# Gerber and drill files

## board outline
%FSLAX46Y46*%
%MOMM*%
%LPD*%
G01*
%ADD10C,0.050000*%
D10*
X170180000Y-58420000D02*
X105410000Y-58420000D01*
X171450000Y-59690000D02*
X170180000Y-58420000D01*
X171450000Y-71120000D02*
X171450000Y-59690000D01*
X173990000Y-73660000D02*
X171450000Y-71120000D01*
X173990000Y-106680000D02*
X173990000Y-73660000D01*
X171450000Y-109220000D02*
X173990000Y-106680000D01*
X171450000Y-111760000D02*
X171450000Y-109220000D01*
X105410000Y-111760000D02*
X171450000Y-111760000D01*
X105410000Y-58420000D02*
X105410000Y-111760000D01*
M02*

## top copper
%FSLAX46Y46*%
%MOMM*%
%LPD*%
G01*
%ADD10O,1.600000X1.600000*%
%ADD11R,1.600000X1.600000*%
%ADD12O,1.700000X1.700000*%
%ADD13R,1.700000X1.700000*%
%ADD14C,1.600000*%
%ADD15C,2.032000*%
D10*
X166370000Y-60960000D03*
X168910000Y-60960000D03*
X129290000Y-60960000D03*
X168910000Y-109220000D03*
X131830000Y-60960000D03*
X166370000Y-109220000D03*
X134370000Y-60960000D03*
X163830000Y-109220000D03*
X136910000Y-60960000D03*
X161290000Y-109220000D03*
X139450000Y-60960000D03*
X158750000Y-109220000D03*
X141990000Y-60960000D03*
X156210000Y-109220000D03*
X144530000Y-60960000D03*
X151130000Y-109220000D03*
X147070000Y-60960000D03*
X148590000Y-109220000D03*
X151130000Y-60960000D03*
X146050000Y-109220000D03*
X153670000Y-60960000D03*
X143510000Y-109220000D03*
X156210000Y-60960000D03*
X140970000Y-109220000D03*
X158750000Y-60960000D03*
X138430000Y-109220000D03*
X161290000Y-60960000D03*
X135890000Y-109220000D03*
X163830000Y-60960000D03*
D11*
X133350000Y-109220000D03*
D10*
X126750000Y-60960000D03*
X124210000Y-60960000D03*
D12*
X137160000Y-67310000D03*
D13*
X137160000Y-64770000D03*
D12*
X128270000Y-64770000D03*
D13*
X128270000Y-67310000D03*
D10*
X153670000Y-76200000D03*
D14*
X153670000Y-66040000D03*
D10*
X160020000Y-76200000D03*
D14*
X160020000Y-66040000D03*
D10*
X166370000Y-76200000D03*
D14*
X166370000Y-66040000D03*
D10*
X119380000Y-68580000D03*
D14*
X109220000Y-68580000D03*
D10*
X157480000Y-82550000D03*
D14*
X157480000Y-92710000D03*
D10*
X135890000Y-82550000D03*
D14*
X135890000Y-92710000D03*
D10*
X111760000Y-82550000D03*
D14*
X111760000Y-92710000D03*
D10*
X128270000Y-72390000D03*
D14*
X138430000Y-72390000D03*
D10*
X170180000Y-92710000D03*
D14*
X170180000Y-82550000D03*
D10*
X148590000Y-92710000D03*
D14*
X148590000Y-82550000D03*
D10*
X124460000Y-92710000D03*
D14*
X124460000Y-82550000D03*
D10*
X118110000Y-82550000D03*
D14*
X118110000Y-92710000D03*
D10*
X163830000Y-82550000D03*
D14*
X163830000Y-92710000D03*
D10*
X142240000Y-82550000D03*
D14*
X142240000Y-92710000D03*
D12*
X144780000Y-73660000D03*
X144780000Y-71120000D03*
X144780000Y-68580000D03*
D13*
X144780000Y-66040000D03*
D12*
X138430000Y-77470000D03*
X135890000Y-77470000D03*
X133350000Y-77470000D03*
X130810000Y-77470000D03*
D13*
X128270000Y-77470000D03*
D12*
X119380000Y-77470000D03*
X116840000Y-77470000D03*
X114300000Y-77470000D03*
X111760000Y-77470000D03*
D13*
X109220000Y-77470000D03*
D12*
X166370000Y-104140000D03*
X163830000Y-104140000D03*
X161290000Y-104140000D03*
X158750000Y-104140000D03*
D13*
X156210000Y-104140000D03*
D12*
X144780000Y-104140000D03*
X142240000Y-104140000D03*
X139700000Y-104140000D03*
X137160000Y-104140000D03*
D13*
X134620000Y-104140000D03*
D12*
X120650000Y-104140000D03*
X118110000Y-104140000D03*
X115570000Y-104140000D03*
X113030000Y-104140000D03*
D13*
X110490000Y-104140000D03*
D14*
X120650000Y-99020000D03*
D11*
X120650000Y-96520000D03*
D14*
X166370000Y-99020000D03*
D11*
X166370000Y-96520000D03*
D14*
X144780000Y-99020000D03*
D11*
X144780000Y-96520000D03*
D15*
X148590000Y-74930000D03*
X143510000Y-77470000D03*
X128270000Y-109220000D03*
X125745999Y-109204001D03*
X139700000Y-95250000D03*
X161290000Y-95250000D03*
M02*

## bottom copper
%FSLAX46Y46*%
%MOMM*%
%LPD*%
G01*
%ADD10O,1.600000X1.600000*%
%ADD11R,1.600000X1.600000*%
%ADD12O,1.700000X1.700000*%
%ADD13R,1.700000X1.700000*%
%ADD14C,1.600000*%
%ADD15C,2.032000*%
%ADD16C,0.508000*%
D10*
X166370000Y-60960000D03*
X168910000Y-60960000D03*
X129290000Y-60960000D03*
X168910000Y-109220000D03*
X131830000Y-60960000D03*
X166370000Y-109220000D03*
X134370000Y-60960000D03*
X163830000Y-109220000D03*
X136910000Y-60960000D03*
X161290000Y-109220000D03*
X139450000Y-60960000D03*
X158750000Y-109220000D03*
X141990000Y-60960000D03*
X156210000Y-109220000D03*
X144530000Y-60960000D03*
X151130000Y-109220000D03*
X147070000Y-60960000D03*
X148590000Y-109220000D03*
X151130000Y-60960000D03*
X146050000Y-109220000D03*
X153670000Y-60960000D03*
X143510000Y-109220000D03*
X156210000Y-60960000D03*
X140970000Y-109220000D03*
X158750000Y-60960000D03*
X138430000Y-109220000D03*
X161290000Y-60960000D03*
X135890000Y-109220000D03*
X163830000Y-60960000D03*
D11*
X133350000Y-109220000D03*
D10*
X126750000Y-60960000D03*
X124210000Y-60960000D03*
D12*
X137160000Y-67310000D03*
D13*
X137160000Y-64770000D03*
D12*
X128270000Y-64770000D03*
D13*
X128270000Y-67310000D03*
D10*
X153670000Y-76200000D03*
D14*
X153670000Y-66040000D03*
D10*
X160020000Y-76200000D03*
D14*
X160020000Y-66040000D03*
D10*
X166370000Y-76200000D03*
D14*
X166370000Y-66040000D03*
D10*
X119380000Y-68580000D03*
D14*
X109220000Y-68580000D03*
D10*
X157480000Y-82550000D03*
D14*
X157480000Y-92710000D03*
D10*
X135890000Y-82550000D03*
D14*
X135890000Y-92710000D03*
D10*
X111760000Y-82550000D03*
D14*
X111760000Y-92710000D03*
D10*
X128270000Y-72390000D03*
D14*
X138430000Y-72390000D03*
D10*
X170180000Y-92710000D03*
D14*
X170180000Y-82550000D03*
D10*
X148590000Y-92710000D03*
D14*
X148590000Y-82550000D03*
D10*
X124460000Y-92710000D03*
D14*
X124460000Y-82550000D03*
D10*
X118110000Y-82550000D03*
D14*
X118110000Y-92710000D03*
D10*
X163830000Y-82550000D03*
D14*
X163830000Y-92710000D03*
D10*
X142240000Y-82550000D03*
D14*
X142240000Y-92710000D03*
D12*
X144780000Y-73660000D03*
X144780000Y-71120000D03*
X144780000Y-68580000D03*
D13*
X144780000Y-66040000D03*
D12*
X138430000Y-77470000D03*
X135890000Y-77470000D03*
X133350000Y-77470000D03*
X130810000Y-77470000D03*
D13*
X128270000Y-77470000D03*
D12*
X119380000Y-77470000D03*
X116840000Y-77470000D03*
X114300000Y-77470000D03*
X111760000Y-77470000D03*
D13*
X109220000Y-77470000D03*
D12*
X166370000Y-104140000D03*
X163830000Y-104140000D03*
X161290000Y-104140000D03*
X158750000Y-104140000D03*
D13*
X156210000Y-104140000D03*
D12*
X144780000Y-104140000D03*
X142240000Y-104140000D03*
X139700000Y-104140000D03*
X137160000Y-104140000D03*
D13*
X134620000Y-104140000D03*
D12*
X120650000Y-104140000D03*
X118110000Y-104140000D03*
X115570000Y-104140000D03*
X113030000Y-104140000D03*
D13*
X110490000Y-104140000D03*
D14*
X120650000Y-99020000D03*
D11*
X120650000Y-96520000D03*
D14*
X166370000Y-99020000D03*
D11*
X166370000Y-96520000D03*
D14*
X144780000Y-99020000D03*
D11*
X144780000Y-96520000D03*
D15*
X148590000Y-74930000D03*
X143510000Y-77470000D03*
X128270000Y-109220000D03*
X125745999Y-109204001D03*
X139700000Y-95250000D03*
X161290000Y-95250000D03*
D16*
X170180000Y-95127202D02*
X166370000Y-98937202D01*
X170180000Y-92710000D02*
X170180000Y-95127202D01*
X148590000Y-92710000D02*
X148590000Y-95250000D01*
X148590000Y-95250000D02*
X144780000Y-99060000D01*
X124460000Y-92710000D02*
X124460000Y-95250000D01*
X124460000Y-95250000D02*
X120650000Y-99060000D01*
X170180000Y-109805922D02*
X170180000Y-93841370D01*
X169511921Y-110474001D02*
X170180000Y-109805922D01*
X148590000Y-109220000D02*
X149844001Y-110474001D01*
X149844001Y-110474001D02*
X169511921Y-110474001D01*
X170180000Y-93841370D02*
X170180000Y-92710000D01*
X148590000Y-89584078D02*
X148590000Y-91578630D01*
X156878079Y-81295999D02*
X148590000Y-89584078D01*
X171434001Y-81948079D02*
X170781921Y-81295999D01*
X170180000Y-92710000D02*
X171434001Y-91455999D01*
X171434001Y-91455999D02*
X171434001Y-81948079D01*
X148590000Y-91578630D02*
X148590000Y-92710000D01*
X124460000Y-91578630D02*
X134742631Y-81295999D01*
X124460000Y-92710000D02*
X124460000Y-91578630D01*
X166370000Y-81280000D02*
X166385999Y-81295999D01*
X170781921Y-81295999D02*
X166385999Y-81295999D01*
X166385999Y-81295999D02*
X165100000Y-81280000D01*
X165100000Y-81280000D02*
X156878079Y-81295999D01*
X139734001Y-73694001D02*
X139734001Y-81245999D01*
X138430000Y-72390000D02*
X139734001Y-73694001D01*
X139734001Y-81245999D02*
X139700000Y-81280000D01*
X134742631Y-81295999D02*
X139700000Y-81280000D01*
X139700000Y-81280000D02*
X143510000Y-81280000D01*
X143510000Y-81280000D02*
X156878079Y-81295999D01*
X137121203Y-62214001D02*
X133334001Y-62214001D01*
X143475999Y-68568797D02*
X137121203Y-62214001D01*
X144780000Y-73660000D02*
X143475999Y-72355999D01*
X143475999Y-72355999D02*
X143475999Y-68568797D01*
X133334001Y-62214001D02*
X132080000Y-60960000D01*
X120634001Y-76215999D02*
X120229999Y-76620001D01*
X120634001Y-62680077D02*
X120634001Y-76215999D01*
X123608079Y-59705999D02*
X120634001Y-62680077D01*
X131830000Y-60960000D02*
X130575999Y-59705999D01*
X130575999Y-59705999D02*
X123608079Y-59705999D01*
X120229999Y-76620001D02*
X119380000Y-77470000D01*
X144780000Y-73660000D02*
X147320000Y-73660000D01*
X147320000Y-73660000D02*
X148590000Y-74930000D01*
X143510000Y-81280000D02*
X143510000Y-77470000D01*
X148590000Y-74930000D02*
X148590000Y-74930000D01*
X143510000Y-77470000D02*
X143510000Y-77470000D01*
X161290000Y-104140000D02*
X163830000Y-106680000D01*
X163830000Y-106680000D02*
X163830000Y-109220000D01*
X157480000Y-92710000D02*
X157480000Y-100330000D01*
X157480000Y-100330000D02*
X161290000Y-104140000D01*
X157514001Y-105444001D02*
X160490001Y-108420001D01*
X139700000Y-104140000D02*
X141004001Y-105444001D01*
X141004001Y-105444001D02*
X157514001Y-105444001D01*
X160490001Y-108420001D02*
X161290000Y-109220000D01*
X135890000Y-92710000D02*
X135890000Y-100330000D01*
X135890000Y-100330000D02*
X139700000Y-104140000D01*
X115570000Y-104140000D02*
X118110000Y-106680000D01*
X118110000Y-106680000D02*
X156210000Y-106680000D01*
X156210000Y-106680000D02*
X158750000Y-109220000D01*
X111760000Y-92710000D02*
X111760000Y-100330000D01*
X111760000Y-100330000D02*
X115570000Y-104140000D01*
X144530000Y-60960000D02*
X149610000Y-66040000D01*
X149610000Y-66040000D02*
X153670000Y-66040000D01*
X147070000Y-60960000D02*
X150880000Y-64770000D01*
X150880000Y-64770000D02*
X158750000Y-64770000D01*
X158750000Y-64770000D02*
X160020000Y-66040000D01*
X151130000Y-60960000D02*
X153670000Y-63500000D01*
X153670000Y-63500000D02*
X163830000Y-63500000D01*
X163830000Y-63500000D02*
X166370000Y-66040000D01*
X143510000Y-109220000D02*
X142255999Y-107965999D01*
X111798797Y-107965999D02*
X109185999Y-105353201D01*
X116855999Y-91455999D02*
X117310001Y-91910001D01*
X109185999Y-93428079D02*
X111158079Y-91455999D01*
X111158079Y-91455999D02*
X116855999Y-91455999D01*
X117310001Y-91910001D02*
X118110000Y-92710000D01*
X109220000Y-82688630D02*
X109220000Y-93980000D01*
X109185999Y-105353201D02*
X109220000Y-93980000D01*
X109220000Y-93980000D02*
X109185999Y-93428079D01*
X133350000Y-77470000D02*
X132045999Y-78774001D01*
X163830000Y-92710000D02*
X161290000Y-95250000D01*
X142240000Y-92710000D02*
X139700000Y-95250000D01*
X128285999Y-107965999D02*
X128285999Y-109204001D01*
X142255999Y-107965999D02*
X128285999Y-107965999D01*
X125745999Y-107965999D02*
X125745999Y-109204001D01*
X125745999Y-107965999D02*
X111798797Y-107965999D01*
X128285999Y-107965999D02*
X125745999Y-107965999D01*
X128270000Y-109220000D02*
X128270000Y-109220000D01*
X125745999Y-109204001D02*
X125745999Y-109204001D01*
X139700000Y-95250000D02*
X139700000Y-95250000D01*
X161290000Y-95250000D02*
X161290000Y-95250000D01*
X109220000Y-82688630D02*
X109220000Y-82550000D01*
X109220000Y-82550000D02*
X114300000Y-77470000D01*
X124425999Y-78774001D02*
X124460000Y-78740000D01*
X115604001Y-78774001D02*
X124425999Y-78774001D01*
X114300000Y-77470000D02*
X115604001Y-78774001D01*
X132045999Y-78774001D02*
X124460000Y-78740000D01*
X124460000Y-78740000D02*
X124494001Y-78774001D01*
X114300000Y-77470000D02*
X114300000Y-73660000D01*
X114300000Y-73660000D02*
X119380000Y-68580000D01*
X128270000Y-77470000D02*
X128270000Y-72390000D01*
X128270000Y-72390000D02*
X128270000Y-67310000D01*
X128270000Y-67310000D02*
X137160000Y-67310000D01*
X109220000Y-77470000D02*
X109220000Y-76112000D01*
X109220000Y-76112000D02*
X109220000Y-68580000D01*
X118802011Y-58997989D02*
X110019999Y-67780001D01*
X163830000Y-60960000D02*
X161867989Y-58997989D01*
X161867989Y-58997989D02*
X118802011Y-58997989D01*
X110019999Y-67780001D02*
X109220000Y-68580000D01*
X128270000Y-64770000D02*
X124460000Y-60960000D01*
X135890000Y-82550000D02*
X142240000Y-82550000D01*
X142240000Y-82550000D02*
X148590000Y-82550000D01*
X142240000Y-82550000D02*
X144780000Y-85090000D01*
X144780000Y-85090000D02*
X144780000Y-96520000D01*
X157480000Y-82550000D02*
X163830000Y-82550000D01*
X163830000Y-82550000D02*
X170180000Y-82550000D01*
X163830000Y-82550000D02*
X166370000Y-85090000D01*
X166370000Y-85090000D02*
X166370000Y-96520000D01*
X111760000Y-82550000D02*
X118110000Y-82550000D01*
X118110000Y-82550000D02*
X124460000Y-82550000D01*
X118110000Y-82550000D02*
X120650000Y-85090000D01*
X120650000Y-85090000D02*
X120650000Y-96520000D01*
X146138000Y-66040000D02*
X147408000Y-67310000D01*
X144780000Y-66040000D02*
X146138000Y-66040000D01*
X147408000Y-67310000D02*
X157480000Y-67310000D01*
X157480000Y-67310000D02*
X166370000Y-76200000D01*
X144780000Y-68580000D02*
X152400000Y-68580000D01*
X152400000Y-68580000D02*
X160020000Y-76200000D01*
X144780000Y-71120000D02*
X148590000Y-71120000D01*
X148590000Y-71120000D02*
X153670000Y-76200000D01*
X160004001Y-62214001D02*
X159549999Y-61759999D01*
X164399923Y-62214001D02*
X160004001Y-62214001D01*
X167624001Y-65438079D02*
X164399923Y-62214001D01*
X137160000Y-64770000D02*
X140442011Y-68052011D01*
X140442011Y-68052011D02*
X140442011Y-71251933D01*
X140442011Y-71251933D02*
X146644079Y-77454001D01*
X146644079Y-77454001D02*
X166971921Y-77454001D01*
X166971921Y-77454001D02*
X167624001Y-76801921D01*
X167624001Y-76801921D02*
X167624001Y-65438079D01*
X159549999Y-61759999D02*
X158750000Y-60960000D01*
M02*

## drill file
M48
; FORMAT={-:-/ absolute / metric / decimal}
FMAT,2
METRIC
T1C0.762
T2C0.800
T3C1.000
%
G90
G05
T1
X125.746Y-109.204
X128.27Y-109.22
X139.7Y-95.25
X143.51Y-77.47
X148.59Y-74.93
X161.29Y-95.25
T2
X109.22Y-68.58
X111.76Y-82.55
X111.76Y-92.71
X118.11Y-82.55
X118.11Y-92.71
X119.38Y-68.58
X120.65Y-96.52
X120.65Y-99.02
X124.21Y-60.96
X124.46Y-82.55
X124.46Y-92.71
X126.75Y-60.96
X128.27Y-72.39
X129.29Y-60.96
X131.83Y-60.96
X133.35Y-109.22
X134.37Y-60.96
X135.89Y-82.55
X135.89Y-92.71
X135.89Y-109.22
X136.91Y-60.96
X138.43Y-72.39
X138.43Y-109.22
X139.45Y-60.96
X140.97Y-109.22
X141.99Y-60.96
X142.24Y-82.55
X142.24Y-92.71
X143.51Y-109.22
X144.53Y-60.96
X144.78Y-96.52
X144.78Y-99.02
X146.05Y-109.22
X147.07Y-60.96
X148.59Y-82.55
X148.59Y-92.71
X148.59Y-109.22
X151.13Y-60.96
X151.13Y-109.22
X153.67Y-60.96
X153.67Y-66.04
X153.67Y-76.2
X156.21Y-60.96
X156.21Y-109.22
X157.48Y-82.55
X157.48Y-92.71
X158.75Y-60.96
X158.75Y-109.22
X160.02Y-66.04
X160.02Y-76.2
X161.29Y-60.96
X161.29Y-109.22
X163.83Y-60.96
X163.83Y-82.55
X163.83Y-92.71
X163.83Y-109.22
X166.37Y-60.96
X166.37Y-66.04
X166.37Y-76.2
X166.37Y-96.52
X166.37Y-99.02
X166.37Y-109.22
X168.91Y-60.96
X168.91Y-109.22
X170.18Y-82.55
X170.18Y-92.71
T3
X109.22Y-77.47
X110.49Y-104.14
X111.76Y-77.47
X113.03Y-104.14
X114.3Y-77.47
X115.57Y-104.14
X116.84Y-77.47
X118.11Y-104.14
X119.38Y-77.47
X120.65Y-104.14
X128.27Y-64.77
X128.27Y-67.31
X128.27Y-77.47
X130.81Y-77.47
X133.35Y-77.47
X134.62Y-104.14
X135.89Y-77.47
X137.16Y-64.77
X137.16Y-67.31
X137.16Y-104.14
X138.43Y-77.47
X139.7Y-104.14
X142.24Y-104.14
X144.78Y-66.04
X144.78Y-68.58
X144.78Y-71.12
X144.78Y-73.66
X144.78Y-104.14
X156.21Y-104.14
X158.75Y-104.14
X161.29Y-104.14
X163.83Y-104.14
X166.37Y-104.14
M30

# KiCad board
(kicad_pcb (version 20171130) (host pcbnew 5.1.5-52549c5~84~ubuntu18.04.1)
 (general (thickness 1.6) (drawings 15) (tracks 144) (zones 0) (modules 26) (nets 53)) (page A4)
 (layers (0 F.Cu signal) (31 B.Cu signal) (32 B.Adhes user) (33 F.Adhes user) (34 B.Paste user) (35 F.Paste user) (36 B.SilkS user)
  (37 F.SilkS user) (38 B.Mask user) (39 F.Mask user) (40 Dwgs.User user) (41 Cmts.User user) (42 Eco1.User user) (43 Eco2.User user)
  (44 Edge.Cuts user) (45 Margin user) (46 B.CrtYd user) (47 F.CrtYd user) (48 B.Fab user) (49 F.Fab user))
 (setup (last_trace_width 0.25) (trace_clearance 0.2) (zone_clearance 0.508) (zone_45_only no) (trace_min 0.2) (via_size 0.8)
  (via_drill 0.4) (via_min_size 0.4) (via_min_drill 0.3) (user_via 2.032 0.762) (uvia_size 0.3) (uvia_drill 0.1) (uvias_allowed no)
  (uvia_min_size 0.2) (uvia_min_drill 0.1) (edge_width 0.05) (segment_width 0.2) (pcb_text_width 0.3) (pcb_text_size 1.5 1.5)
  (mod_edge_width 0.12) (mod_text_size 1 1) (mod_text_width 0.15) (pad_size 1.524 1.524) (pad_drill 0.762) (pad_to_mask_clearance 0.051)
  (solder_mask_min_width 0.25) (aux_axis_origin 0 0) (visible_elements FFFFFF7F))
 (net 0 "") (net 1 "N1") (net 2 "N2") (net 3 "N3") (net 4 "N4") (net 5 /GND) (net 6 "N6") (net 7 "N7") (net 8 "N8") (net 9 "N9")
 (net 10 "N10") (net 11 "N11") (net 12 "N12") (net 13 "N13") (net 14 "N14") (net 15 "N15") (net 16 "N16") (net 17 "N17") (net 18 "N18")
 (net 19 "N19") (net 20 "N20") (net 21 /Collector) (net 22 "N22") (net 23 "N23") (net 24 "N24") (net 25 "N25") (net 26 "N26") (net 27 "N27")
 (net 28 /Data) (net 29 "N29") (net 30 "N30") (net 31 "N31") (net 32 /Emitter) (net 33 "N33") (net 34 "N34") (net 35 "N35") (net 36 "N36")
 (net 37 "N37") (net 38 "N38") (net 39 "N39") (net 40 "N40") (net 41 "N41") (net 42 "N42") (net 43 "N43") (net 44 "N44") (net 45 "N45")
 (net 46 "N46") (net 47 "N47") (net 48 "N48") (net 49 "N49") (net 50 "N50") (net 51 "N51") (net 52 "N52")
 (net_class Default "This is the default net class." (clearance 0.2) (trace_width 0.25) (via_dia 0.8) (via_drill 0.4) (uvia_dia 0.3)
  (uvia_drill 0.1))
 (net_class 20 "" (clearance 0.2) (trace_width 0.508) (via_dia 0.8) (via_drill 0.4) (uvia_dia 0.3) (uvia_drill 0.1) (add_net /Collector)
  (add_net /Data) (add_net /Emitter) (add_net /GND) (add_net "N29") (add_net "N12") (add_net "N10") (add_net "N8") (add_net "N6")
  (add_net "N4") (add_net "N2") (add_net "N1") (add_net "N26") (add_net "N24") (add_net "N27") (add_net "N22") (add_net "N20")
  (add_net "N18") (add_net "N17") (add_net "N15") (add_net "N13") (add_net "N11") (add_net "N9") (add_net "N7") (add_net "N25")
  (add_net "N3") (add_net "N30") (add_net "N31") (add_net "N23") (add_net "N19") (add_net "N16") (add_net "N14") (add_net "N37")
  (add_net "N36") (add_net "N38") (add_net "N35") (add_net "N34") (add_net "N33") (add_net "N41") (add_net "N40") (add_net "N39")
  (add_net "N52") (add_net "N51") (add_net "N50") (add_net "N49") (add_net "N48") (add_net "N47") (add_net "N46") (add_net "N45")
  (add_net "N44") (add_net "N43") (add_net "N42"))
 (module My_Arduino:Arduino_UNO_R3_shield (layer F.Cu) (at 133.35 109.22)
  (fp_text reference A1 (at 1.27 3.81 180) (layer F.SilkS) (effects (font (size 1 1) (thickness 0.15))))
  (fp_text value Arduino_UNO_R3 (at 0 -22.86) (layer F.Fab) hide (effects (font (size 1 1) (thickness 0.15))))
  (pad 16 thru_hole oval (at 33.02 -48.26 270) (size 1.6 1.6) (drill 0.8) (layers *.Cu *.Mask) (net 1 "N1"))
  (pad 15 thru_hole oval (at 35.56 -48.26 270) (size 1.6 1.6) (drill 0.8) (layers *.Cu *.Mask) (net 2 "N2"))
  (pad 30 thru_hole oval (at -4.06 -48.26 270) (size 1.6 1.6) (drill 0.8) (layers *.Cu *.Mask) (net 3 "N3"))
  (pad 14 thru_hole oval (at 35.56 0 270) (size 1.6 1.6) (drill 0.8) (layers *.Cu *.Mask) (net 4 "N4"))
  (pad 29 thru_hole oval (at -1.52 -48.26 270) (size 1.6 1.6) (drill 0.8) (layers *.Cu *.Mask) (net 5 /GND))
  (pad 13 thru_hole oval (at 33.02 0 270) (size 1.6 1.6) (drill 0.8) (layers *.Cu *.Mask) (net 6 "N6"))
  (pad 28 thru_hole oval (at 1.02 -48.26 270) (size 1.6 1.6) (drill 0.8) (layers *.Cu *.Mask) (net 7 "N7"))
  (pad 12 thru_hole oval (at 30.48 0 270) (size 1.6 1.6) (drill 0.8) (layers *.Cu *.Mask) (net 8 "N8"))
  (pad 27 thru_hole oval (at 3.56 -48.26 270) (size 1.6 1.6) (drill 0.8) (layers *.Cu *.Mask) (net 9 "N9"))
  (pad 11 thru_hole oval (at 27.94 0 270) (size 1.6 1.6) (drill 0.8) (layers *.Cu *.Mask) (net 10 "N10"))
  (pad 26 thru_hole oval (at 6.1 -48.26 270) (size 1.6 1.6) (drill 0.8) (layers *.Cu *.Mask) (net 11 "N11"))
  (pad 10 thru_hole oval (at 25.4 0 270) (size 1.6 1.6) (drill 0.8) (layers *.Cu *.Mask) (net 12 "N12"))
  (pad 25 thru_hole oval (at 8.64 -48.26 270) (size 1.6 1.6) (drill 0.8) (layers *.Cu *.Mask) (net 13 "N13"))
  (pad 9 thru_hole oval (at 22.86 0 270) (size 1.6 1.6) (drill 0.8) (layers *.Cu *.Mask) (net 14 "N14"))
  (pad 24 thru_hole oval (at 11.18 -48.26 270) (size 1.6 1.6) (drill 0.8) (layers *.Cu *.Mask) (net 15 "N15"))
  (pad 8 thru_hole oval (at 17.78 0 270) (size 1.6 1.6) (drill 0.8) (layers *.Cu *.Mask) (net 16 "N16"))
  (pad 23 thru_hole oval (at 13.72 -48.26 270) (size 1.6 1.6) (drill 0.8) (layers *.Cu *.Mask) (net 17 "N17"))
  (pad 7 thru_hole oval (at 15.24 0 270) (size 1.6 1.6) (drill 0.8) (layers *.Cu *.Mask) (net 5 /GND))
  (pad 22 thru_hole oval (at 17.78 -48.26 270) (size 1.6 1.6) (drill 0.8) (layers *.Cu *.Mask) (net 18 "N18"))
  (pad 6 thru_hole oval (at 12.7 0 270) (size 1.6 1.6) (drill 0.8) (layers *.Cu *.Mask) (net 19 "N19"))
  (pad 21 thru_hole oval (at 20.32 -48.26 270) (size 1.6 1.6) (drill 0.8) (layers *.Cu *.Mask) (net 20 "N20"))
  (pad 5 thru_hole oval (at 10.16 0 270) (size 1.6 1.6) (drill 0.8) (layers *.Cu *.Mask) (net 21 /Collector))
  (pad 20 thru_hole oval (at 22.86 -48.26 270) (size 1.6 1.6) (drill 0.8) (layers *.Cu *.Mask) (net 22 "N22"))
  (pad 4 thru_hole oval (at 7.62 0 270) (size 1.6 1.6) (drill 0.8) (layers *.Cu *.Mask) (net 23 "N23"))
  (pad 19 thru_hole oval (at 25.4 -48.26 270) (size 1.6 1.6) (drill 0.8) (layers *.Cu *.Mask) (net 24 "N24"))
  (pad 3 thru_hole oval (at 5.08 0 270) (size 1.6 1.6) (drill 0.8) (layers *.Cu *.Mask) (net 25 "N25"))
  (pad 18 thru_hole oval (at 27.94 -48.26 270) (size 1.6 1.6) (drill 0.8) (layers *.Cu *.Mask) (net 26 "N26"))
  (pad 2 thru_hole oval (at 2.54 0 270) (size 1.6 1.6) (drill 0.8) (layers *.Cu *.Mask) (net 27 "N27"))
  (pad 17 thru_hole oval (at 30.48 -48.26 270) (size 1.6 1.6) (drill 0.8) (layers *.Cu *.Mask) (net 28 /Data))
  (pad 1 thru_hole rect (at 0 0 270) (size 1.6 1.6) (drill 0.8) (layers *.Cu *.Mask) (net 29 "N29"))
  (pad 31 thru_hole oval (at -6.6 -48.26 270) (size 1.6 1.6) (drill 0.8) (layers *.Cu *.Mask) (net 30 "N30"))
  (pad 32 thru_hole oval (at -9.14 -48.26 270) (size 1.6 1.6) (drill 0.8) (layers *.Cu *.Mask) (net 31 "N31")))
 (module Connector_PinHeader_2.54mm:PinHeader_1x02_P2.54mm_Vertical (layer F.Cu) (at 137.16 64.77)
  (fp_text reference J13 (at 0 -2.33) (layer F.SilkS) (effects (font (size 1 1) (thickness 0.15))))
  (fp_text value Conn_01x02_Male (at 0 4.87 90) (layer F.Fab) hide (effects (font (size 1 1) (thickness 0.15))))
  (pad 2 thru_hole oval (at 0 2.54) (size 1.7 1.7) (drill 1) (layers *.Cu *.Mask) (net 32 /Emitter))
  (pad 1 thru_hole rect (at 0 0) (size 1.7 1.7) (drill 1) (layers *.Cu *.Mask) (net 24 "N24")))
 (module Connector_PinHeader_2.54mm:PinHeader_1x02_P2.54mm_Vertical (layer F.Cu) (at 128.27 67.31 180)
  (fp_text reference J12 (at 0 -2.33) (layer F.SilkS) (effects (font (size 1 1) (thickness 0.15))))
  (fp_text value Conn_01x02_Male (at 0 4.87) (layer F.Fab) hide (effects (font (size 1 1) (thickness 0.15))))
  (pad 2 thru_hole oval (at 0 2.54 180) (size 1.7 1.7) (drill 1) (layers *.Cu *.Mask) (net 31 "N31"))
  (pad 1 thru_hole rect (at 0 0 180) (size 1.7 1.7) (drill 1) (layers *.Cu *.Mask) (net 32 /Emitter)))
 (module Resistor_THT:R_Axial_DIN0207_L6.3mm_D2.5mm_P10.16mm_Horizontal (layer F.Cu) (at 153.67 66.04 270)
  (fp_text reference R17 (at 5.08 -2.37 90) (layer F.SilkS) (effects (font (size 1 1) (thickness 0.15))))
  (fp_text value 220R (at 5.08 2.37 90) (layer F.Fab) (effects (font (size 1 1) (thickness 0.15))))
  (pad 2 thru_hole oval (at 10.16 0 270) (size 1.6 1.6) (drill 0.8) (layers *.Cu *.Mask) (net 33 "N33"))
  (pad 1 thru_hole circle (at 0 0 270) (size 1.6 1.6) (drill 0.8) (layers *.Cu *.Mask) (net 15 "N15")))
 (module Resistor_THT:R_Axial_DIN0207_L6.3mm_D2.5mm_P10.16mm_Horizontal (layer F.Cu) (at 160.02 66.04 270)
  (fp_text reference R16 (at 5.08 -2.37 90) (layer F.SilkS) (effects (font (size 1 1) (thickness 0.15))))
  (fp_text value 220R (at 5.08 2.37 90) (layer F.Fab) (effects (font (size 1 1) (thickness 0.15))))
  (pad 2 thru_hole oval (at 10.16 0 270) (size 1.6 1.6) (drill 0.8) (layers *.Cu *.Mask) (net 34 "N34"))
  (pad 1 thru_hole circle (at 0 0 270) (size 1.6 1.6) (drill 0.8) (layers *.Cu *.Mask) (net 17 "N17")))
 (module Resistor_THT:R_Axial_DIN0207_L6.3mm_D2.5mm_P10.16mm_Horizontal (layer F.Cu) (at 166.37 66.04 270)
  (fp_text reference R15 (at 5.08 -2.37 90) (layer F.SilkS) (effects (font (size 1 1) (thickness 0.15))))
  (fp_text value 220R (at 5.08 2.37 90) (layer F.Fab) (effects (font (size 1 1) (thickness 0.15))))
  (pad 2 thru_hole oval (at 10.16 0 270) (size 1.6 1.6) (drill 0.8) (layers *.Cu *.Mask) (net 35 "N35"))
  (pad 1 thru_hole circle (at 0 0 270) (size 1.6 1.6) (drill 0.8) (layers *.Cu *.Mask) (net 18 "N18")))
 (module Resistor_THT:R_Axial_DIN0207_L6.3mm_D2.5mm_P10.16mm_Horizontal (layer F.Cu) (at 109.22 68.58)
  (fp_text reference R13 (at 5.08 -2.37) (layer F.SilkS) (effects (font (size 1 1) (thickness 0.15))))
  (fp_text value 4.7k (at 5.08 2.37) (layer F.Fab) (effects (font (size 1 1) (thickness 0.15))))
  (pad 2 thru_hole oval (at 10.16 0) (size 1.6 1.6) (drill 0.8) (layers *.Cu *.Mask) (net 21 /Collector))
  (pad 1 thru_hole circle (at 0 0) (size 1.6 1.6) (drill 0.8) (layers *.Cu *.Mask) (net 28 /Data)))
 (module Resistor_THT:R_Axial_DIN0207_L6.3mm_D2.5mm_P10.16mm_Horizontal (layer F.Cu) (at 157.48 92.71 90)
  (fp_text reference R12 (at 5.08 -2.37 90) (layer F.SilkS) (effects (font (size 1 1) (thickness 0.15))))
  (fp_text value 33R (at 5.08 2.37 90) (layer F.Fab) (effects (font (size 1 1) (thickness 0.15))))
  (pad 2 thru_hole oval (at 10.16 0 90) (size 1.6 1.6) (drill 0.8) (layers *.Cu *.Mask) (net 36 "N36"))
  (pad 1 thru_hole circle (at 0 0 90) (size 1.6 1.6) (drill 0.8) (layers *.Cu *.Mask) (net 8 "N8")))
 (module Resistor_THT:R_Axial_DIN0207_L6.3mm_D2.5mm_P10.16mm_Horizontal (layer F.Cu) (at 135.89 92.71 90)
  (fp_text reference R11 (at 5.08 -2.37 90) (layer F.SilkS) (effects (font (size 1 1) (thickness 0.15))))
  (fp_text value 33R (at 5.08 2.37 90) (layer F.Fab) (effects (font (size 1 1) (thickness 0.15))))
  (pad 2 thru_hole oval (at 10.16 0 90) (size 1.6 1.6) (drill 0.8) (layers *.Cu *.Mask) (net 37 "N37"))
  (pad 1 thru_hole circle (at 0 0 90) (size 1.6 1.6) (drill 0.8) (layers *.Cu *.Mask) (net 10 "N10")))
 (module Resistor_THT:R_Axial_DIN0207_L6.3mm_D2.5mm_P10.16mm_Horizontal (layer F.Cu) (at 111.76 92.71 90)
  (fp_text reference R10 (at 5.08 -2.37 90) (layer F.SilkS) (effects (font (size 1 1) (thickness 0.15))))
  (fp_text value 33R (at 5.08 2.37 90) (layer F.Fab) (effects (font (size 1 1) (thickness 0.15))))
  (pad 2 thru_hole oval (at 10.16 0 90) (size 1.6 1.6) (drill 0.8) (layers *.Cu *.Mask) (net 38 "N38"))
  (pad 1 thru_hole circle (at 0 0 90) (size 1.6 1.6) (drill 0.8) (layers *.Cu *.Mask) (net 12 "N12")))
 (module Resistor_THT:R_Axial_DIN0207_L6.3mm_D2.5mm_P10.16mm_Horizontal (layer F.Cu) (at 138.43 72.39 180)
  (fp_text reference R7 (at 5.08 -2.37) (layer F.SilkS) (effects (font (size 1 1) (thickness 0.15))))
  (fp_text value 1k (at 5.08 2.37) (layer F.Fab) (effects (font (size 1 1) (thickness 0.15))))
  (pad 2 thru_hole oval (at 10.16 0 180) (size 1.6 1.6) (drill 0.8) (layers *.Cu *.Mask) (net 32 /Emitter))
  (pad 1 thru_hole circle (at 0 0 180) (size 1.6 1.6) (drill 0.8) (layers *.Cu *.Mask) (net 5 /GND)))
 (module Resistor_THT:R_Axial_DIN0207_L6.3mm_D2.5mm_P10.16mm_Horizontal (layer F.Cu) (at 170.18 82.55 270)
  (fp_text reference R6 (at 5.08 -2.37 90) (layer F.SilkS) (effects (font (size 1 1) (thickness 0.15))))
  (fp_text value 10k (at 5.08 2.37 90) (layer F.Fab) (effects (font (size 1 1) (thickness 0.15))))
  (pad 2 thru_hole oval (at 10.16 0 270) (size 1.6 1.6) (drill 0.8) (layers *.Cu *.Mask) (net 5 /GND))
  (pad 1 thru_hole circle (at 0 0 270) (size 1.6 1.6) (drill 0.8) (layers *.Cu *.Mask) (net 36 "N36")))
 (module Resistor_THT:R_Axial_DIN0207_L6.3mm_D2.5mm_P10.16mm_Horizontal (layer F.Cu) (at 148.59 82.55 270)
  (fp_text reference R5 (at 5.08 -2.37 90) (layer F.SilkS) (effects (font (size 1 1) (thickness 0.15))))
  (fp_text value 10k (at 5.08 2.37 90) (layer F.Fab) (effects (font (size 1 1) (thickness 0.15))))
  (pad 2 thru_hole oval (at 10.16 0 270) (size 1.6 1.6) (drill 0.8) (layers *.Cu *.Mask) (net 5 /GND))
  (pad 1 thru_hole circle (at 0 0 270) (size 1.6 1.6) (drill 0.8) (layers *.Cu *.Mask) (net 37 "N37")))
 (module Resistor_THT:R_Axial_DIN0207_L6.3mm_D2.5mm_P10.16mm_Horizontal (layer F.Cu) (at 124.46 82.55 270)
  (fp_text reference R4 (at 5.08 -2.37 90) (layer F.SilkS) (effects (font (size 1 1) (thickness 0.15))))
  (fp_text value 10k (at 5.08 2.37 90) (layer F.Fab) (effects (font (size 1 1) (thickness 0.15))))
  (pad 2 thru_hole oval (at 10.16 0 270) (size 1.6 1.6) (drill 0.8) (layers *.Cu *.Mask) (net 5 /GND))
  (pad 1 thru_hole circle (at 0 0 270) (size 1.6 1.6) (drill 0.8) (layers *.Cu *.Mask) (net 38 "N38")))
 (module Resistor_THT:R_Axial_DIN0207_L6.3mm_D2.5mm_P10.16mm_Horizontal (layer F.Cu) (at 118.11 92.71 90)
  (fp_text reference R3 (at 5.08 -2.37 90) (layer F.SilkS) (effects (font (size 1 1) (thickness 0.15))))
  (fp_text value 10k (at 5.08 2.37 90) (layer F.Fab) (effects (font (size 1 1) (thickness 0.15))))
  (pad 2 thru_hole oval (at 10.16 0 90) (size 1.6 1.6) (drill 0.8) (layers *.Cu *.Mask) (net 38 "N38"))
  (pad 1 thru_hole circle (at 0 0 90) (size 1.6 1.6) (drill 0.8) (layers *.Cu *.Mask) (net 21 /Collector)))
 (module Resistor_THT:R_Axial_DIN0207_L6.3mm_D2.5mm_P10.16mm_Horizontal (layer F.Cu) (at 163.83 92.71 90)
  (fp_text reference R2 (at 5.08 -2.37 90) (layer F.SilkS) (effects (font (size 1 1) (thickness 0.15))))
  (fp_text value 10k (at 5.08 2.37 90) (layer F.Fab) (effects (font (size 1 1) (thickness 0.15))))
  (pad 2 thru_hole oval (at 10.16 0 90) (size 1.6 1.6) (drill 0.8) (layers *.Cu *.Mask) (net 36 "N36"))
  (pad 1 thru_hole circle (at 0 0 90) (size 1.6 1.6) (drill 0.8) (layers *.Cu *.Mask) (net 21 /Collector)))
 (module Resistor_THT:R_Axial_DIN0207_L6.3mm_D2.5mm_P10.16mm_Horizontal (layer F.Cu) (at 142.24 92.71 90)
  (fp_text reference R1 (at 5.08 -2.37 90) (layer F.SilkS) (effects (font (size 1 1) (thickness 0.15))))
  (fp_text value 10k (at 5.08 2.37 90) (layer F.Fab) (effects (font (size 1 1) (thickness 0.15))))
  (pad 2 thru_hole oval (at 10.16 0 90) (size 1.6 1.6) (drill 0.8) (layers *.Cu *.Mask) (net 37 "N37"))
  (pad 1 thru_hole circle (at 0 0 90) (size 1.6 1.6) (drill 0.8) (layers *.Cu *.Mask) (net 21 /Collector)))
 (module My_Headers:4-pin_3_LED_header (layer F.Cu) (at 144.78 66.04)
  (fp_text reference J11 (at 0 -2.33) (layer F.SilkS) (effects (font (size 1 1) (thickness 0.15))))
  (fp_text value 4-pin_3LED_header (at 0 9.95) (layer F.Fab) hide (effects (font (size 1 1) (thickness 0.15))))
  (pad 4 thru_hole oval (at 0 7.62) (size 1.7 1.7) (drill 1) (layers *.Cu *.Mask) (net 5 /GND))
  (pad 3 thru_hole oval (at 0 5.08) (size 1.7 1.7) (drill 1) (layers *.Cu *.Mask) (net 33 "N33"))
  (pad 2 thru_hole oval (at 0 2.54) (size 1.7 1.7) (drill 1) (layers *.Cu *.Mask) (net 34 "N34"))
  (pad 1 thru_hole rect (at 0 0) (size 1.7 1.7) (drill 1) (layers *.Cu *.Mask) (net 35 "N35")))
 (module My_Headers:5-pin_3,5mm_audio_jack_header (layer F.Cu) (at 128.27 77.47 90)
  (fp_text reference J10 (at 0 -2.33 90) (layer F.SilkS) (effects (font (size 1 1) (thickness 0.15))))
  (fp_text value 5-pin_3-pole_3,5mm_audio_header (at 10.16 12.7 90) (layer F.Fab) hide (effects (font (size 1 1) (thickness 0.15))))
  (pad 5 thru_hole oval (at 0 10.16 90) (size 1.7 1.7) (drill 1) (layers *.Cu *.Mask) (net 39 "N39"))
  (pad 4 thru_hole oval (at 0 7.62 90) (size 1.7 1.7) (drill 1) (layers *.Cu *.Mask) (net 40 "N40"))
  (pad 3 thru_hole oval (at 0 5.08 90) (size 1.7 1.7) (drill 1) (layers *.Cu *.Mask) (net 21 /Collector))
  (pad 2 thru_hole oval (at 0 2.54 90) (size 1.7 1.7) (drill 1) (layers *.Cu *.Mask) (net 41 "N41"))
  (pad 1 thru_hole rect (at 0 0 90) (size 1.7 1.7) (drill 1) (layers *.Cu *.Mask) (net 32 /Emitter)))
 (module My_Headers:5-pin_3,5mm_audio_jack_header (layer F.Cu) (at 109.22 77.47 90)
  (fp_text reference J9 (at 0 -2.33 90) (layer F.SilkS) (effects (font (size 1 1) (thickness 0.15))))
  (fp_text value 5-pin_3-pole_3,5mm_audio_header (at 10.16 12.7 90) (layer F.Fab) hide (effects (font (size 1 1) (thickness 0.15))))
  (pad 5 thru_hole oval (at 0 10.16 90) (size 1.7 1.7) (drill 1) (layers *.Cu *.Mask) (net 5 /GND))
  (pad 4 thru_hole oval (at 0 7.62 90) (size 1.7 1.7) (drill 1) (layers *.Cu *.Mask) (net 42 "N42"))
  (pad 3 thru_hole oval (at 0 5.08 90) (size 1.7 1.7) (drill 1) (layers *.Cu *.Mask) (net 21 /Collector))
  (pad 2 thru_hole oval (at 0 2.54 90) (size 1.7 1.7) (drill 1) (layers *.Cu *.Mask) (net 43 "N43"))
  (pad 1 thru_hole rect (at 0 0 90) (size 1.7 1.7) (drill 1) (layers *.Cu *.Mask) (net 28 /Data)))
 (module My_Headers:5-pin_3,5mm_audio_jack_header (layer F.Cu) (at 156.21 104.14 90)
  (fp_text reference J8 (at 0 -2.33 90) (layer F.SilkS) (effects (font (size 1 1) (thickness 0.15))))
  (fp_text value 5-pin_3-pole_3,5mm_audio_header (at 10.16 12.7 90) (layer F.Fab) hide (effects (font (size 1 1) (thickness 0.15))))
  (pad 5 thru_hole oval (at 0 10.16 90) (size 1.7 1.7) (drill 1) (layers *.Cu *.Mask) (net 36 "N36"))
  (pad 4 thru_hole oval (at 0 7.62 90) (size 1.7 1.7) (drill 1) (layers *.Cu *.Mask) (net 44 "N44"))
  (pad 3 thru_hole oval (at 0 5.08 90) (size 1.7 1.7) (drill 1) (layers *.Cu *.Mask) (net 8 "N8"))
  (pad 2 thru_hole oval (at 0 2.54 90) (size 1.7 1.7) (drill 1) (layers *.Cu *.Mask) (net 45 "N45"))
  (pad 1 thru_hole rect (at 0 0 90) (size 1.7 1.7) (drill 1) (layers *.Cu *.Mask) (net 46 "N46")))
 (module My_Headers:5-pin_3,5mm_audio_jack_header (layer F.Cu) (at 134.62 104.14 90)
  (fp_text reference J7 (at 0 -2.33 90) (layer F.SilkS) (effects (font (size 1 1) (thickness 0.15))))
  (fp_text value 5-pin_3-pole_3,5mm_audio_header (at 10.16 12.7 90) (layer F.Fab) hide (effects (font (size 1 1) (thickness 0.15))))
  (pad 5 thru_hole oval (at 0 10.16 90) (size 1.7 1.7) (drill 1) (layers *.Cu *.Mask) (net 37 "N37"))
  (pad 4 thru_hole oval (at 0 7.62 90) (size 1.7 1.7) (drill 1) (layers *.Cu *.Mask) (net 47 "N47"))
  (pad 3 thru_hole oval (at 0 5.08 90) (size 1.7 1.7) (drill 1) (layers *.Cu *.Mask) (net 10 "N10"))
  (pad 2 thru_hole oval (at 0 2.54 90) (size 1.7 1.7) (drill 1) (layers *.Cu *.Mask) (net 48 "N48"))
  (pad 1 thru_hole rect (at 0 0 90) (size 1.7 1.7) (drill 1) (layers *.Cu *.Mask) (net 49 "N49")))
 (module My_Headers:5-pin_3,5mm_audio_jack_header (layer F.Cu) (at 110.49 104.14 90)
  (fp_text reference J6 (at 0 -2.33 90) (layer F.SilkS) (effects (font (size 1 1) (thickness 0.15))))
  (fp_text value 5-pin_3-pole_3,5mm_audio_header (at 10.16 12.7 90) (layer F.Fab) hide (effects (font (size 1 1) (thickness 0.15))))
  (pad 5 thru_hole oval (at 0 10.16 90) (size 1.7 1.7) (drill 1) (layers *.Cu *.Mask) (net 38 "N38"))
  (pad 4 thru_hole oval (at 0 7.62 90) (size 1.7 1.7) (drill 1) (layers *.Cu *.Mask) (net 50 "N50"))
  (pad 3 thru_hole oval (at 0 5.08 90) (size 1.7 1.7) (drill 1) (layers *.Cu *.Mask) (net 12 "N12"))
  (pad 2 thru_hole oval (at 0 2.54 90) (size 1.7 1.7) (drill 1) (layers *.Cu *.Mask) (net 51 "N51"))
  (pad 1 thru_hole rect (at 0 0 90) (size 1.7 1.7) (drill 1) (layers *.Cu *.Mask) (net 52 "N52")))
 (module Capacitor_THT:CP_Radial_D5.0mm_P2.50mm (layer F.Cu) (at 120.65 96.52 270)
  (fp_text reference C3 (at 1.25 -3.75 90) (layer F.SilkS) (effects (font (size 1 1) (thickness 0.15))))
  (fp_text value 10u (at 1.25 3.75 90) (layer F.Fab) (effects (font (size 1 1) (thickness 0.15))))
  (pad 2 thru_hole circle (at 2.5 0 270) (size 1.6 1.6) (drill 0.8) (layers *.Cu *.Mask) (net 5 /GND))
  (pad 1 thru_hole rect (at 0 0 270) (size 1.6 1.6) (drill 0.8) (layers *.Cu *.Mask) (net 38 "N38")))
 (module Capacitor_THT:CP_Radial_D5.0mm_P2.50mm (layer F.Cu) (at 166.37 96.52 270)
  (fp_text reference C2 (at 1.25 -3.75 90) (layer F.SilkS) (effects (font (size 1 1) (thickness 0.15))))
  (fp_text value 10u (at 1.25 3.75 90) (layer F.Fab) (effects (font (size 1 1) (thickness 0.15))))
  (pad 2 thru_hole circle (at 2.5 0 270) (size 1.6 1.6) (drill 0.8) (layers *.Cu *.Mask) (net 5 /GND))
  (pad 1 thru_hole rect (at 0 0 270) (size 1.6 1.6) (drill 0.8) (layers *.Cu *.Mask) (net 36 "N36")))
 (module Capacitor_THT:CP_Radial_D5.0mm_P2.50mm (layer F.Cu) (at 144.78 96.52 270)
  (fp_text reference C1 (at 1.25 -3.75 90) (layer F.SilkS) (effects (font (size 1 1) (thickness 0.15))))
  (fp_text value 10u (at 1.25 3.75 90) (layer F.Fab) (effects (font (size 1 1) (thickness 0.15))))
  (pad 2 thru_hole circle (at 2.5 0 270) (size 1.6 1.6) (drill 0.8) (layers *.Cu *.Mask) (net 5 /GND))
  (pad 1 thru_hole rect (at 0 0 270) (size 1.6 1.6) (drill 0.8) (layers *.Cu *.Mask) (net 37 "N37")))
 (gr_line (start 170.18 58.42) (end 105.41 58.42) (layer Edge.Cuts) (width 0.05))
 (gr_line (start 171.45 59.69) (end 170.18 58.42) (layer Edge.Cuts) (width 0.05))
 (gr_line (start 171.45 71.12) (end 171.45 59.69) (layer Edge.Cuts) (width 0.05))
 (gr_line (start 173.99 73.66) (end 171.45 71.12) (layer Edge.Cuts) (width 0.05))
 (gr_line (start 173.99 106.68) (end 173.99 73.66) (layer Edge.Cuts) (width 0.05))
 (gr_line (start 171.45 109.22) (end 173.99 106.68) (layer Edge.Cuts) (width 0.05))
 (gr_line (start 171.45 111.76) (end 171.45 109.22) (layer Edge.Cuts) (width 0.05))
 (gr_line (start 105.41 111.76) (end 171.45 111.76) (layer Edge.Cuts) (width 0.05))
 (gr_line (start 105.41 58.42) (end 105.41 111.76) (layer Edge.Cuts) (width 0.05))
 (segment (start 170.18 95.127202) (end 166.37 98.937202) (width 0.508) (layer B.Cu) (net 5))
 (segment (start 170.18 92.71) (end 170.18 95.127202) (width 0.508) (layer B.Cu) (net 5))
 (segment (start 148.59 92.71) (end 148.59 95.25) (width 0.508) (layer B.Cu) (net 5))
 (segment (start 148.59 95.25) (end 144.78 99.06) (width 0.508) (layer B.Cu) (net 5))
 (segment (start 124.46 92.71) (end 124.46 95.25) (width 0.508) (layer B.Cu) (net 5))
 (segment (start 124.46 95.25) (end 120.65 99.06) (width 0.508) (layer B.Cu) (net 5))
 (segment (start 170.18 109.805922) (end 170.18 93.84137) (width 0.508) (layer B.Cu) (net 5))
 (segment (start 169.511921 110.474001) (end 170.18 109.805922) (width 0.508) (layer B.Cu) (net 5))
 (segment (start 148.59 109.22) (end 149.844001 110.474001) (width 0.508) (layer B.Cu) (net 5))
 (segment (start 149.844001 110.474001) (end 169.511921 110.474001) (width 0.508) (layer B.Cu) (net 5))
 (segment (start 170.18 93.84137) (end 170.18 92.71) (width 0.508) (layer B.Cu) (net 5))
 (segment (start 148.59 89.584078) (end 148.59 91.57863) (width 0.508) (layer B.Cu) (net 5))
 (segment (start 156.878079 81.295999) (end 148.59 89.584078) (width 0.508) (layer B.Cu) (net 5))
 (segment (start 171.434001 81.948079) (end 170.781921 81.295999) (width 0.508) (layer B.Cu) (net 5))
 (segment (start 170.18 92.71) (end 171.434001 91.455999) (width 0.508) (layer B.Cu) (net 5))
 (segment (start 171.434001 91.455999) (end 171.434001 81.948079) (width 0.508) (layer B.Cu) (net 5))
 (segment (start 148.59 91.57863) (end 148.59 92.71) (width 0.508) (layer B.Cu) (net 5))
 (segment (start 124.46 91.57863) (end 134.742631 81.295999) (width 0.508) (layer B.Cu) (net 5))
 (segment (start 124.46 92.71) (end 124.46 91.57863) (width 0.508) (layer B.Cu) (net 5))
 (segment (start 166.37 81.28) (end 166.385999 81.295999) (width 0.508) (layer B.Cu) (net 5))
 (segment (start 170.781921 81.295999) (end 166.385999 81.295999) (width 0.508) (layer B.Cu) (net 5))
 (segment (start 166.385999 81.295999) (end 165.1 81.28) (width 0.508) (layer B.Cu) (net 5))
 (segment (start 165.1 81.28) (end 156.878079 81.295999) (width 0.508) (layer B.Cu) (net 5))
 (segment (start 139.734001 73.694001) (end 139.734001 81.245999) (width 0.508) (layer B.Cu) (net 5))
 (segment (start 138.43 72.39) (end 139.734001 73.694001) (width 0.508) (layer B.Cu) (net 5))
 (segment (start 139.734001 81.245999) (end 139.7 81.28) (width 0.508) (layer B.Cu) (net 5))
 (segment (start 134.742631 81.295999) (end 139.7 81.28) (width 0.508) (layer B.Cu) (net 5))
 (segment (start 139.7 81.28) (end 143.51 81.28) (width 0.508) (layer B.Cu) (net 5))
 (segment (start 143.51 81.28) (end 156.878079 81.295999) (width 0.508) (layer B.Cu) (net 5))
 (segment (start 137.121203 62.214001) (end 133.334001 62.214001) (width 0.508) (layer B.Cu) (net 5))
 (segment (start 143.475999 68.568797) (end 137.121203 62.214001) (width 0.508) (layer B.Cu) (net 5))
 (segment (start 144.78 73.66) (end 143.475999 72.355999) (width 0.508) (layer B.Cu) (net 5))
 (segment (start 143.475999 72.355999) (end 143.475999 68.568797) (width 0.508) (layer B.Cu) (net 5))
 (segment (start 133.334001 62.214001) (end 132.08 60.96) (width 0.508) (layer B.Cu) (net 5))
 (segment (start 120.634001 76.215999) (end 120.229999 76.620001) (width 0.508) (layer B.Cu) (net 5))
 (segment (start 120.634001 62.680077) (end 120.634001 76.215999) (width 0.508) (layer B.Cu) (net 5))
 (segment (start 123.608079 59.705999) (end 120.634001 62.680077) (width 0.508) (layer B.Cu) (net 5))
 (segment (start 131.83 60.96) (end 130.575999 59.705999) (width 0.508) (layer B.Cu) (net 5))
 (segment (start 130.575999 59.705999) (end 123.608079 59.705999) (width 0.508) (layer B.Cu) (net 5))
 (segment (start 120.229999 76.620001) (end 119.38 77.47) (width 0.508) (layer B.Cu) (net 5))
 (segment (start 144.78 73.66) (end 147.32 73.66) (width 0.508) (layer B.Cu) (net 5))
 (segment (start 147.32 73.66) (end 148.59 74.93) (width 0.508) (layer B.Cu) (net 5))
 (segment (start 143.51 81.28) (end 143.51 77.47) (width 0.508) (layer B.Cu) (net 5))
 (segment (start 148.59 74.93) (end 148.59 74.93) (width 0.508) (layer B.Cu) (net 5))
 (via (at 148.59 74.93) (size 2.032) (drill 0.762) (layers F.Cu B.Cu) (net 5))
 (segment (start 143.51 77.47) (end 143.51 77.47) (width 0.508) (layer B.Cu) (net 5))
 (via (at 143.51 77.47) (size 2.032) (drill 0.762) (layers F.Cu B.Cu) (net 5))
 (segment (start 161.29 104.14) (end 163.83 106.68) (width 0.508) (layer B.Cu) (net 8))
 (segment (start 163.83 106.68) (end 163.83 109.22) (width 0.508) (layer B.Cu) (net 8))
 (segment (start 157.48 92.71) (end 157.48 100.33) (width 0.508) (layer B.Cu) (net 8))
 (segment (start 157.48 100.33) (end 161.29 104.14) (width 0.508) (layer B.Cu) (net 8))
 (segment (start 157.514001 105.444001) (end 160.490001 108.420001) (width 0.508) (layer B.Cu) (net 10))
 (segment (start 139.7 104.14) (end 141.004001 105.444001) (width 0.508) (layer B.Cu) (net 10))
 (segment (start 141.004001 105.444001) (end 157.514001 105.444001) (width 0.508) (layer B.Cu) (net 10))
 (segment (start 160.490001 108.420001) (end 161.29 109.22) (width 0.508) (layer B.Cu) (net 10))
 (segment (start 135.89 92.71) (end 135.89 100.33) (width 0.508) (layer B.Cu) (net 10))
 (segment (start 135.89 100.33) (end 139.7 104.14) (width 0.508) (layer B.Cu) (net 10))
 (segment (start 115.57 104.14) (end 118.11 106.68) (width 0.508) (layer B.Cu) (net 12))
 (segment (start 118.11 106.68) (end 156.21 106.68) (width 0.508) (layer B.Cu) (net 12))
 (segment (start 156.21 106.68) (end 158.75 109.22) (width 0.508) (layer B.Cu) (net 12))
 (segment (start 111.76 92.71) (end 111.76 100.33) (width 0.508) (layer B.Cu) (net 12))
 (segment (start 111.76 100.33) (end 115.57 104.14) (width 0.508) (layer B.Cu) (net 12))
 (segment (start 144.53 60.96) (end 149.61 66.04) (width 0.508) (layer B.Cu) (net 15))
 (segment (start 149.61 66.04) (end 153.67 66.04) (width 0.508) (layer B.Cu) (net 15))
 (segment (start 147.07 60.96) (end 150.88 64.77) (width 0.508) (layer B.Cu) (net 17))
 (segment (start 150.88 64.77) (end 158.75 64.77) (width 0.508) (layer B.Cu) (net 17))
 (segment (start 158.75 64.77) (end 160.02 66.04) (width 0.508) (layer B.Cu) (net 17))
 (segment (start 151.13 60.96) (end 153.67 63.5) (width 0.508) (layer B.Cu) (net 18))
 (segment (start 153.67 63.5) (end 163.83 63.5) (width 0.508) (layer B.Cu) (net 18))
 (segment (start 163.83 63.5) (end 166.37 66.04) (width 0.508) (layer B.Cu) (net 18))
 (segment (start 143.51 109.22) (end 142.255999 107.965999) (width 0.508) (layer B.Cu) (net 21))
 (segment (start 111.798797 107.965999) (end 109.185999 105.353201) (width 0.508) (layer B.Cu) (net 21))
 (segment (start 116.855999 91.455999) (end 117.310001 91.910001) (width 0.508) (layer B.Cu) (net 21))
 (segment (start 109.185999 93.428079) (end 111.158079 91.455999) (width 0.508) (layer B.Cu) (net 21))
 (segment (start 111.158079 91.455999) (end 116.855999 91.455999) (width 0.508) (layer B.Cu) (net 21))
 (segment (start 117.310001 91.910001) (end 118.11 92.71) (width 0.508) (layer B.Cu) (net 21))
 (segment (start 109.22 82.68863) (end 109.22 93.98) (width 0.508) (layer B.Cu) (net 21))
 (segment (start 109.185999 105.353201) (end 109.22 93.98) (width 0.508) (layer B.Cu) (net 21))
 (segment (start 109.22 93.98) (end 109.185999 93.428079) (width 0.508) (layer B.Cu) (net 21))
 (segment (start 133.35 77.47) (end 132.045999 78.774001) (width 0.508) (layer B.Cu) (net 21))
 (segment (start 163.83 92.71) (end 161.29 95.25) (width 0.508) (layer B.Cu) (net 21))
 (segment (start 142.24 92.71) (end 139.7 95.25) (width 0.508) (layer B.Cu) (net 21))
 (segment (start 128.285999 107.965999) (end 128.285999 109.204001) (width 0.508) (layer B.Cu) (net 21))
 (segment (start 142.255999 107.965999) (end 128.285999 107.965999) (width 0.508) (layer B.Cu) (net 21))
 (segment (start 125.745999 107.965999) (end 125.745999 109.204001) (width 0.508) (layer B.Cu) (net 21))
 (segment (start 125.745999 107.965999) (end 111.798797 107.965999) (width 0.508) (layer B.Cu) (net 21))
 (segment (start 128.285999 107.965999) (end 125.745999 107.965999) (width 0.508) (layer B.Cu) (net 21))
 (segment (start 128.27 109.22) (end 128.27 109.22) (width 0.508) (layer B.Cu) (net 21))
 (via (at 128.27 109.22) (size 2.032) (drill 0.762) (layers F.Cu B.Cu) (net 21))
 (segment (start 125.745999 109.204001) (end 125.745999 109.204001) (width 0.508) (layer B.Cu) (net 21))
 (via (at 125.745999 109.204001) (size 2.032) (drill 0.762) (layers F.Cu B.Cu) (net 21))
 (segment (start 139.7 95.25) (end 139.7 95.25) (width 0.508) (layer B.Cu) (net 21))
 (via (at 139.7 95.25) (size 2.032) (drill 0.762) (layers F.Cu B.Cu) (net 21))
 (segment (start 161.29 95.25) (end 161.29 95.25) (width 0.508) (layer B.Cu) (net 21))
 (via (at 161.29 95.25) (size 2.032) (drill 0.762) (layers F.Cu B.Cu) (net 21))
 (segment (start 109.22 82.68863) (end 109.22 82.55) (width 0.508) (layer B.Cu) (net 21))
 (segment (start 109.22 82.55) (end 114.3 77.47) (width 0.508) (layer B.Cu) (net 21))
 (segment (start 124.425999 78.774001) (end 124.46 78.74) (width 0.508) (layer B.Cu) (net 21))
 (segment (start 115.604001 78.774001) (end 124.425999 78.774001) (width 0.508) (layer B.Cu) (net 21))
 (segment (start 114.3 77.47) (end 115.604001 78.774001) (width 0.508) (layer B.Cu) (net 21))
 (segment (start 132.045999 78.774001) (end 124.46 78.74) (width 0.508) (layer B.Cu) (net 21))
 (segment (start 124.46 78.74) (end 124.494001 78.774001) (width 0.508) (layer B.Cu) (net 21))
 (segment (start 114.3 77.47) (end 114.3 73.66) (width 0.508) (layer B.Cu) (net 21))
 (segment (start 114.3 73.66) (end 119.38 68.58) (width 0.508) (layer B.Cu) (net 21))
 (segment (start 128.27 77.47) (end 128.27 72.39) (width 0.508) (layer B.Cu) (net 32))
 (segment (start 128.27 72.39) (end 128.27 67.31) (width 0.508) (layer B.Cu) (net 32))
 (segment (start 128.27 67.31) (end 137.16 67.31) (width 0.508) (layer B.Cu) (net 32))
 (segment (start 109.22 77.47) (end 109.22 76.112) (width 0.508) (layer B.Cu) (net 28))
 (segment (start 109.22 76.112) (end 109.22 68.58) (width 0.508) (layer B.Cu) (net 28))
 (segment (start 118.802011 58.997989) (end 110.019999 67.780001) (width 0.508) (layer B.Cu) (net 28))
 (segment (start 163.83 60.96) (end 161.867989 58.997989) (width 0.508) (layer B.Cu) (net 28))
 (segment (start 161.867989 58.997989) (end 118.802011 58.997989) (width 0.508) (layer B.Cu) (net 28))
 (segment (start 110.019999 67.780001) (end 109.22 68.58) (width 0.508) (layer B.Cu) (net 28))
 (segment (start 128.27 64.77) (end 124.46 60.96) (width 0.508) (layer B.Cu) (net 31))
 (segment (start 135.89 82.55) (end 142.24 82.55) (width 0.508) (layer B.Cu) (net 37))
 (segment (start 142.24 82.55) (end 148.59 82.55) (width 0.508) (layer B.Cu) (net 37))
 (segment (start 142.24 82.55) (end 144.78 85.09) (width 0.508) (layer B.Cu) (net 37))
 (segment (start 144.78 85.09) (end 144.78 96.52) (width 0.508) (layer B.Cu) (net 37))
 (segment (start 157.48 82.55) (end 163.83 82.55) (width 0.508) (layer B.Cu) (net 36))
 (segment (start 163.83 82.55) (end 170.18 82.55) (width 0.508) (layer B.Cu) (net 36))
 (segment (start 163.83 82.55) (end 166.37 85.09) (width 0.508) (layer B.Cu) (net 36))
 (segment (start 166.37 85.09) (end 166.37 96.52) (width 0.508) (layer B.Cu) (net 36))
 (segment (start 111.76 82.55) (end 118.11 82.55) (width 0.508) (layer B.Cu) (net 38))
 (segment (start 118.11 82.55) (end 124.46 82.55) (width 0.508) (layer B.Cu) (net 38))
 (segment (start 118.11 82.55) (end 120.65 85.09) (width 0.508) (layer B.Cu) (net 38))
 (segment (start 120.65 85.09) (end 120.65 96.52) (width 0.508) (layer B.Cu) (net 38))
 (segment (start 146.138 66.04) (end 147.408 67.31) (width 0.508) (layer B.Cu) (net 35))
 (segment (start 144.78 66.04) (end 146.138 66.04) (width 0.508) (layer B.Cu) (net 35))
 (segment (start 147.408 67.31) (end 157.48 67.31) (width 0.508) (layer B.Cu) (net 35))
 (segment (start 157.48 67.31) (end 166.37 76.2) (width 0.508) (layer B.Cu) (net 35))
 (segment (start 144.78 68.58) (end 152.4 68.58) (width 0.508) (layer B.Cu) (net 34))
 (segment (start 152.4 68.58) (end 160.02 76.2) (width 0.508) (layer B.Cu) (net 34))
 (segment (start 144.78 71.12) (end 148.59 71.12) (width 0.508) (layer B.Cu) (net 33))
 (segment (start 148.59 71.12) (end 153.67 76.2) (width 0.508) (layer B.Cu) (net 33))
 (segment (start 160.004001 62.214001) (end 159.549999 61.759999) (width 0.508) (layer B.Cu) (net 24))
 (segment (start 164.399923 62.214001) (end 160.004001 62.214001) (width 0.508) (layer B.Cu) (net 24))
 (segment (start 167.624001 65.438079) (end 164.399923 62.214001) (width 0.508) (layer B.Cu) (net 24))
 (segment (start 137.16 64.77) (end 140.442011 68.052011) (width 0.508) (layer B.Cu) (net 24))
 (segment (start 140.442011 68.052011) (end 140.442011 71.251933) (width 0.508) (layer B.Cu) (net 24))
 (segment (start 140.442011 71.251933) (end 146.644079 77.454001) (width 0.508) (layer B.Cu) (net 24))
 (segment (start 146.644079 77.454001) (end 166.971921 77.454001) (width 0.508) (layer B.Cu) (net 24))
 (segment (start 166.971921 77.454001) (end 167.624001 76.801921) (width 0.508) (layer B.Cu) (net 24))
 (segment (start 167.624001 76.801921) (end 167.624001 65.438079) (width 0.508) (layer B.Cu) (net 24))
 (segment (start 159.549999 61.759999) (end 158.75 60.96) (width 0.508) (layer B.Cu) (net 24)))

